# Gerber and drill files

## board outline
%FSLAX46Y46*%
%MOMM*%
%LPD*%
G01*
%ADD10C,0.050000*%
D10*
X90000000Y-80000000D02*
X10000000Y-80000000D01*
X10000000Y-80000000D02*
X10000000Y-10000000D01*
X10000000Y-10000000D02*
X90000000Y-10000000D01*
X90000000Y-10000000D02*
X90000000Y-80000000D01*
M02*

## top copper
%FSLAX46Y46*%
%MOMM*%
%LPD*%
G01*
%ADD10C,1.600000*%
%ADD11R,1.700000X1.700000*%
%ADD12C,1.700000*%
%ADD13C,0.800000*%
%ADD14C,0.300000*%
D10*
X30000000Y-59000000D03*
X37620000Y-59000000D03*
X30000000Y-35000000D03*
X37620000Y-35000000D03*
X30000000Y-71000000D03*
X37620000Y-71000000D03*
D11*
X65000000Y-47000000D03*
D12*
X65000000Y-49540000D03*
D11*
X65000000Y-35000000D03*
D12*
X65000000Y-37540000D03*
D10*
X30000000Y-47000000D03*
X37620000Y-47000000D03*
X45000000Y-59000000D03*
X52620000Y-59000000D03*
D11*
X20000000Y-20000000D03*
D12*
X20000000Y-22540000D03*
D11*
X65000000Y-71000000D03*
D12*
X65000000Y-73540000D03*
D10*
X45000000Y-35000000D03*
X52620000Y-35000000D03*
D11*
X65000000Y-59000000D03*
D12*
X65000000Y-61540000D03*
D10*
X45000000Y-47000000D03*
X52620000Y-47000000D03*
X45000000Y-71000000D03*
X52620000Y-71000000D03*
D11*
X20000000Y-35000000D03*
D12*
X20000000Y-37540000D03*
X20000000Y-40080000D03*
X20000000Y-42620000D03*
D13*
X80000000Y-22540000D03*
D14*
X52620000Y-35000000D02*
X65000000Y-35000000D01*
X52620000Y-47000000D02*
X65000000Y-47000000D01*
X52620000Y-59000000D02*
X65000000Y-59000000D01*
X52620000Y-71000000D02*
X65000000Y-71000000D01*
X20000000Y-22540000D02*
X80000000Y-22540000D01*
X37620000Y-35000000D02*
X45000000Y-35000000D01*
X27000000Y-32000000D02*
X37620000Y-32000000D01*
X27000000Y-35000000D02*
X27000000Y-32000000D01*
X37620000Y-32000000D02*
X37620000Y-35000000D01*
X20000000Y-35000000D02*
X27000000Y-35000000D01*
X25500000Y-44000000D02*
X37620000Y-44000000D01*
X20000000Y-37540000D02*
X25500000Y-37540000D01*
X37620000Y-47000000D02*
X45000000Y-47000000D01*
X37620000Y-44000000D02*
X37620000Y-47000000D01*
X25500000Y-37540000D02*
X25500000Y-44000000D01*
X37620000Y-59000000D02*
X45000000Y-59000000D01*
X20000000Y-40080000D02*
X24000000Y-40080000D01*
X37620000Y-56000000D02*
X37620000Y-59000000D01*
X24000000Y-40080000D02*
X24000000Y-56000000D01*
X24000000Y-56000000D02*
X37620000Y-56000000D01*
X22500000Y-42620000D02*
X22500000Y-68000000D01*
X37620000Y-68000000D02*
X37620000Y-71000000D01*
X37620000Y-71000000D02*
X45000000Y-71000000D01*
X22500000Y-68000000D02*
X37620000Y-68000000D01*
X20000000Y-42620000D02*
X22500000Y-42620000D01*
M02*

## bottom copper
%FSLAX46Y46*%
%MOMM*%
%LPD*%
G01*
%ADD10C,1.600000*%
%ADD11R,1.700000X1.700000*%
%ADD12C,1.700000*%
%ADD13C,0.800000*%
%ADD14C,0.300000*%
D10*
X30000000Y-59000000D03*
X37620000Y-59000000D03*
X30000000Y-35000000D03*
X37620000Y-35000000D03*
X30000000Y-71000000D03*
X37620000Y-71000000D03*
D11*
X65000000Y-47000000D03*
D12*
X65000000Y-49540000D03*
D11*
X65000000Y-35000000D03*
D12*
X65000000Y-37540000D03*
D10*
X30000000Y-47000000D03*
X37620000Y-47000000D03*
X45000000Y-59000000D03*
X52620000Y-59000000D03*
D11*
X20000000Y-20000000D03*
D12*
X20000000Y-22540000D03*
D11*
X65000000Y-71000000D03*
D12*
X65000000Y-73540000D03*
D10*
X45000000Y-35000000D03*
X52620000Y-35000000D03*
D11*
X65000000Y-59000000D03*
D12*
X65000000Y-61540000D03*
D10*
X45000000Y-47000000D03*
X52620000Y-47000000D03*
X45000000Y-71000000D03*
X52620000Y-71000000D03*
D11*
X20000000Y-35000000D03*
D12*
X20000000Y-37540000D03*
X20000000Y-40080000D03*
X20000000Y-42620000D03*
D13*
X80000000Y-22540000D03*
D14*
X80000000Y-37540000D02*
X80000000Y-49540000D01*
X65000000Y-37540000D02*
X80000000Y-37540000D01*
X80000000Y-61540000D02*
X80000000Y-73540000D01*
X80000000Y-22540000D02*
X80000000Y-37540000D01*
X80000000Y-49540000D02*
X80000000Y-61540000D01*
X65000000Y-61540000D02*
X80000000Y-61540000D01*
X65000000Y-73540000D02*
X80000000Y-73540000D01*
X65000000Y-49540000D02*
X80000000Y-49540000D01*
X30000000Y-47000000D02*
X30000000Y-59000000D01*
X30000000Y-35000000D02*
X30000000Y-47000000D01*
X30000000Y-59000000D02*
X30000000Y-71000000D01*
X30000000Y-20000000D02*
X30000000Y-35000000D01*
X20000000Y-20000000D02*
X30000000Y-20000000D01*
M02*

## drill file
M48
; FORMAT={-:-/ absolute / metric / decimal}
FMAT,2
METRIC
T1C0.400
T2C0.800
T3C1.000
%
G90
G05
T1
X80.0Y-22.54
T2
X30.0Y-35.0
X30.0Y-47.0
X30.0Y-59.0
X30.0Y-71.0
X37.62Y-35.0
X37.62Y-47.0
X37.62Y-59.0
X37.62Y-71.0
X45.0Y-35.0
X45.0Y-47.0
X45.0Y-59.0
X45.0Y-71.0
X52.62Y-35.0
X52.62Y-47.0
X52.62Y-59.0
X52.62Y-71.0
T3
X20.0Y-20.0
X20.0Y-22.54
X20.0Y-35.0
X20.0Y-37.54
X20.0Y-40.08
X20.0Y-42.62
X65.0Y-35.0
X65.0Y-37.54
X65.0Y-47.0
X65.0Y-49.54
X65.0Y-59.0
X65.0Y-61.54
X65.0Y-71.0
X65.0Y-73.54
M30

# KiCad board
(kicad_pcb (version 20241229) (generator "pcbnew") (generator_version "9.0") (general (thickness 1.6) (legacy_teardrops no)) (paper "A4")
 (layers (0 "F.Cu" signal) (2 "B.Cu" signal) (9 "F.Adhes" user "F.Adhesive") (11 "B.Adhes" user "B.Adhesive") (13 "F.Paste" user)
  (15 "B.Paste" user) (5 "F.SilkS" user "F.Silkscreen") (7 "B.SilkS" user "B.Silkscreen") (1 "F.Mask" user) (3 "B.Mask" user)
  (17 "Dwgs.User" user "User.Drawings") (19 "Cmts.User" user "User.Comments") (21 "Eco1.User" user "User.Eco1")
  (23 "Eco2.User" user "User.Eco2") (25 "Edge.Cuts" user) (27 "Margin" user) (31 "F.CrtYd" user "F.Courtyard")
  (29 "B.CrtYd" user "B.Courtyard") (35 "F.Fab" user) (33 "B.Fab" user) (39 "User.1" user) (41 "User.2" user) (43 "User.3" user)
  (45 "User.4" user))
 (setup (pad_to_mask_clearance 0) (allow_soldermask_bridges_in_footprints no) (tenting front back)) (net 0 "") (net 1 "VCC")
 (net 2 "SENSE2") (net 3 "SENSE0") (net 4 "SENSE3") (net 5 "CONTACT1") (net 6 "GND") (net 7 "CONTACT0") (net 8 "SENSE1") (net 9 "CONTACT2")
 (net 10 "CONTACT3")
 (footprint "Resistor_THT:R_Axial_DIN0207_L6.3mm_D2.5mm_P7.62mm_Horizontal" (layer "F.Cu") (at 30 59)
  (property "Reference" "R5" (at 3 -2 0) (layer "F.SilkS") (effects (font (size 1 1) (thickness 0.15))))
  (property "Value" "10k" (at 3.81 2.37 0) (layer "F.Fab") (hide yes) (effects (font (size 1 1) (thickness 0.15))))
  (pad "1" thru_hole circle (at 0 0) (size 1.6 1.6) (drill 0.8) (layers "*.Cu" "*.Mask") (remove_unused_layers no) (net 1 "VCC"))
  (pad "2" thru_hole circle (at 7.62 0) (size 1.6 1.6) (drill 0.8) (layers "*.Cu" "*.Mask") (remove_unused_layers no) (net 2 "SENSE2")))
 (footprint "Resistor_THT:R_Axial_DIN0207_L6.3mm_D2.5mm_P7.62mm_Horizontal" (layer "F.Cu") (at 30 35)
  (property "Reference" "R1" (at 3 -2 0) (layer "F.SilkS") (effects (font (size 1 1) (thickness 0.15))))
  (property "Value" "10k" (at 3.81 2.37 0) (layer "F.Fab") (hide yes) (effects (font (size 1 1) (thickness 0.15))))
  (pad "1" thru_hole circle (at 0 0) (size 1.6 1.6) (drill 0.8) (layers "*.Cu" "*.Mask") (remove_unused_layers no) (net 1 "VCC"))
  (pad "2" thru_hole circle (at 7.62 0) (size 1.6 1.6) (drill 0.8) (layers "*.Cu" "*.Mask") (remove_unused_layers no) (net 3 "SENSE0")))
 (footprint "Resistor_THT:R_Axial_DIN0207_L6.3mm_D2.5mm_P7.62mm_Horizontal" (layer "F.Cu") (at 30 71)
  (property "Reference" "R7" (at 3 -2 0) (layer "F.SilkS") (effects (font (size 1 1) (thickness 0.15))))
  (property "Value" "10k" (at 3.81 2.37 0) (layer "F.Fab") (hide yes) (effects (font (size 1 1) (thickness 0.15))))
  (pad "1" thru_hole circle (at 0 0) (size 1.6 1.6) (drill 0.8) (layers "*.Cu" "*.Mask") (remove_unused_layers no) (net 1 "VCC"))
  (pad "2" thru_hole circle (at 7.62 0) (size 1.6 1.6) (drill 0.8) (layers "*.Cu" "*.Mask") (remove_unused_layers no) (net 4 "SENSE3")))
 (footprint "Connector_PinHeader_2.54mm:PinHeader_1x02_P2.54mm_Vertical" (layer "F.Cu") (at 65 47)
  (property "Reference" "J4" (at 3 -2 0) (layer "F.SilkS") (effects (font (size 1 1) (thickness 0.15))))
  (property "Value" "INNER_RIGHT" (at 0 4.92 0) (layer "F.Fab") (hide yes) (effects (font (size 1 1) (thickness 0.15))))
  (pad "1" thru_hole rect (at 0 0) (size 1.7 1.7) (drill 1) (layers "*.Cu" "*.Mask") (remove_unused_layers no) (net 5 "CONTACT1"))
  (pad "2" thru_hole circle (at 0 2.54) (size 1.7 1.7) (drill 1) (layers "*.Cu" "*.Mask") (remove_unused_layers no) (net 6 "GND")))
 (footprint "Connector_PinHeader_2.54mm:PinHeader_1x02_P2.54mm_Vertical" (layer "F.Cu") (at 65 35)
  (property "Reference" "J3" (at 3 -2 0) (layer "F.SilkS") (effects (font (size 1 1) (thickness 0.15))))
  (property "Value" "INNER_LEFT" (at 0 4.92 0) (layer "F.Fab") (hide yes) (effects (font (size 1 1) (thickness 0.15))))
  (pad "1" thru_hole rect (at 0 0) (size 1.7 1.7) (drill 1) (layers "*.Cu" "*.Mask") (remove_unused_layers no) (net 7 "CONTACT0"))
  (pad "2" thru_hole circle (at 0 2.54) (size 1.7 1.7) (drill 1) (layers "*.Cu" "*.Mask") (remove_unused_layers no) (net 6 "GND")))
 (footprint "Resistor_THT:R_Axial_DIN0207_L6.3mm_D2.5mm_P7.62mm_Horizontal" (layer "F.Cu") (at 30 47)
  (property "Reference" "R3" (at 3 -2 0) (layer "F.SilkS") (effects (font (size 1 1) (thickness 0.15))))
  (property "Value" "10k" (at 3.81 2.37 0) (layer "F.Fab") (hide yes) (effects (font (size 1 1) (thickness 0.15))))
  (pad "1" thru_hole circle (at 0 0) (size 1.6 1.6) (drill 0.8) (layers "*.Cu" "*.Mask") (remove_unused_layers no) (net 1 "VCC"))
  (pad "2" thru_hole circle (at 7.62 0) (size 1.6 1.6) (drill 0.8) (layers "*.Cu" "*.Mask") (remove_unused_layers no) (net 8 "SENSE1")))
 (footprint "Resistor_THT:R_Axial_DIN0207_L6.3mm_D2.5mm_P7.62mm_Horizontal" (layer "F.Cu") (at 45 59)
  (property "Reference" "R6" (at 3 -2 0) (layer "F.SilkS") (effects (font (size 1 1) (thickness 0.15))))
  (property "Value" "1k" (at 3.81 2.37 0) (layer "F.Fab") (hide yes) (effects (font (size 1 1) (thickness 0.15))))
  (pad "1" thru_hole circle (at 0 0) (size 1.6 1.6) (drill 0.8) (layers "*.Cu" "*.Mask") (remove_unused_layers no) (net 2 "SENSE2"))
  (pad "2" thru_hole circle (at 7.62 0) (size 1.6 1.6) (drill 0.8) (layers "*.Cu" "*.Mask") (remove_unused_layers no) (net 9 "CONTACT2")))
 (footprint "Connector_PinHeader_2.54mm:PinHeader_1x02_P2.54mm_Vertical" (layer "F.Cu") (at 20 20)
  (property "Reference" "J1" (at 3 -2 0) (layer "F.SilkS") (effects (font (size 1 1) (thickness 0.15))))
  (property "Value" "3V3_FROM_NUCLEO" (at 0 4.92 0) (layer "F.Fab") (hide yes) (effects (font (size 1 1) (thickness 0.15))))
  (pad "1" thru_hole rect (at 0 0) (size 1.7 1.7) (drill 1) (layers "*.Cu" "*.Mask") (remove_unused_layers no) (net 1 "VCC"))
  (pad "2" thru_hole circle (at 0 2.54) (size 1.7 1.7) (drill 1) (layers "*.Cu" "*.Mask") (remove_unused_layers no) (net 6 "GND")))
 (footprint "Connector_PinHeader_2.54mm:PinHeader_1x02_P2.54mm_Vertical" (layer "F.Cu") (at 65 71)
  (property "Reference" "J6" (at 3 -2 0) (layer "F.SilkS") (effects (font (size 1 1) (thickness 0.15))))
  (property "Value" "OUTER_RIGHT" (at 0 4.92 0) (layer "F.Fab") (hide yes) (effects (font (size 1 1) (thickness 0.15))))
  (pad "1" thru_hole rect (at 0 0) (size 1.7 1.7) (drill 1) (layers "*.Cu" "*.Mask") (remove_unused_layers no) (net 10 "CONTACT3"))
  (pad "2" thru_hole circle (at 0 2.54) (size 1.7 1.7) (drill 1) (layers "*.Cu" "*.Mask") (remove_unused_layers no) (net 6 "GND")))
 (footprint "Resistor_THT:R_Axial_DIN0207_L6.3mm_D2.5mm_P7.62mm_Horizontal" (layer "F.Cu") (at 45 35)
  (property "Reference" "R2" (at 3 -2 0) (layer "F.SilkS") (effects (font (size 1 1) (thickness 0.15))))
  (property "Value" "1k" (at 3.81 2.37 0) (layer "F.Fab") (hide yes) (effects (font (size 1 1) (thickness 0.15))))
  (pad "1" thru_hole circle (at 0 0) (size 1.6 1.6) (drill 0.8) (layers "*.Cu" "*.Mask") (remove_unused_layers no) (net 3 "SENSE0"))
  (pad "2" thru_hole circle (at 7.62 0) (size 1.6 1.6) (drill 0.8) (layers "*.Cu" "*.Mask") (remove_unused_layers no) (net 7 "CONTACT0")))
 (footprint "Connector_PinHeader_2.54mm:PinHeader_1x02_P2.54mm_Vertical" (layer "F.Cu") (at 65 59)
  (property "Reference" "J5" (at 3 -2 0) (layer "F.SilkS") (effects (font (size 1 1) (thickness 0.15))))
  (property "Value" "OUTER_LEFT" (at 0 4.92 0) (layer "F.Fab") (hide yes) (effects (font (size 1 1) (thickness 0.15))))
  (pad "1" thru_hole rect (at 0 0) (size 1.7 1.7) (drill 1) (layers "*.Cu" "*.Mask") (remove_unused_layers no) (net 9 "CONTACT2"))
  (pad "2" thru_hole circle (at 0 2.54) (size 1.7 1.7) (drill 1) (layers "*.Cu" "*.Mask") (remove_unused_layers no) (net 6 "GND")))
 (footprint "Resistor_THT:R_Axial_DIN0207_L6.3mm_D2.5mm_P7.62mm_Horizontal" (layer "F.Cu") (at 45 47)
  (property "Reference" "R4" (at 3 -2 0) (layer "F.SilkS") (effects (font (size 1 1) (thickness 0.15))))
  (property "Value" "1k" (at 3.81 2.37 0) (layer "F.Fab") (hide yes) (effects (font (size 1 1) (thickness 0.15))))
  (pad "1" thru_hole circle (at 0 0) (size 1.6 1.6) (drill 0.8) (layers "*.Cu" "*.Mask") (remove_unused_layers no) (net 8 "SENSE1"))
  (pad "2" thru_hole circle (at 7.62 0) (size 1.6 1.6) (drill 0.8) (layers "*.Cu" "*.Mask") (remove_unused_layers no) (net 5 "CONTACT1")))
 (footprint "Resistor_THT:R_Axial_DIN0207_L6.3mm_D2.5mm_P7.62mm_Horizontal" (layer "F.Cu") (at 45 71)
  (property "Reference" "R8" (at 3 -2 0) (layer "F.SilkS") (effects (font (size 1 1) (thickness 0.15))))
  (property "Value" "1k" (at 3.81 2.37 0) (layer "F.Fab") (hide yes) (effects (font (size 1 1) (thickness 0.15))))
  (pad "1" thru_hole circle (at 0 0) (size 1.6 1.6) (drill 0.8) (layers "*.Cu" "*.Mask") (remove_unused_layers no) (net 4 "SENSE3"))
  (pad "2" thru_hole circle (at 7.62 0) (size 1.6 1.6) (drill 0.8) (layers "*.Cu" "*.Mask") (remove_unused_layers no) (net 10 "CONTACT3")))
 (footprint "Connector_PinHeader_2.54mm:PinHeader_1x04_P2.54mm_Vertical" (layer "F.Cu") (at 20 35)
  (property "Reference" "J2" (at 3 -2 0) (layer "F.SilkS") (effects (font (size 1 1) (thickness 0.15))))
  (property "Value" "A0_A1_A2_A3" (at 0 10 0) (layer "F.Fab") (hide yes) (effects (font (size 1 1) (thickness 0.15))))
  (pad "1" thru_hole rect (at 0 0) (size 1.7 1.7) (drill 1) (layers "*.Cu" "*.Mask") (remove_unused_layers no) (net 3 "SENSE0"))
  (pad "2" thru_hole circle (at 0 2.54) (size 1.7 1.7) (drill 1) (layers "*.Cu" "*.Mask") (remove_unused_layers no) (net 8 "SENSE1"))
  (pad "3" thru_hole circle (at 0 5.08) (size 1.7 1.7) (drill 1) (layers "*.Cu" "*.Mask") (remove_unused_layers no) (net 2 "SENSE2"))
  (pad "4" thru_hole circle (at 0 7.62) (size 1.7 1.7) (drill 1) (layers "*.Cu" "*.Mask") (remove_unused_layers no) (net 4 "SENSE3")))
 (gr_line (start 90 80) (end 10 80) (stroke (width 0.05) (type default)) (layer "Edge.Cuts"))
 (gr_line (start 10 80) (end 10 10) (stroke (width 0.05) (type default)) (layer "Edge.Cuts"))
 (gr_line (start 10 10) (end 90 10) (stroke (width 0.05) (type default)) (layer "Edge.Cuts"))
 (gr_line (start 90 10) (end 90 80) (stroke (width 0.05) (type default)) (layer "Edge.Cuts"))
 (segment (start 52.62 35) (end 65 35) (width 0.3) (layer "F.Cu") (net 7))
 (segment (start 52.62 47) (end 65 47) (width 0.3) (layer "F.Cu") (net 5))
 (segment (start 52.62 59) (end 65 59) (width 0.3) (layer "F.Cu") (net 9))
 (segment (start 52.62 71) (end 65 71) (width 0.3) (layer "F.Cu") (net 10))
 (segment (start 20 22.54) (end 80 22.54) (width 0.3) (layer "F.Cu") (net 6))
 (via (at 80 22.54) (size 0.8) (drill 0.4) (layers "F.Cu" "B.Cu") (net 6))
 (segment (start 80 37.54) (end 80 49.54) (width 0.3) (layer "B.Cu") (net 6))
 (segment (start 65 37.54) (end 80 37.54) (width 0.3) (layer "B.Cu") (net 6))
 (segment (start 80 61.54) (end 80 73.54) (width 0.3) (layer "B.Cu") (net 6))
 (segment (start 80 22.54) (end 80 37.54) (width 0.3) (layer "B.Cu") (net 6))
 (segment (start 80 49.54) (end 80 61.54) (width 0.3) (layer "B.Cu") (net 6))
 (segment (start 65 61.54) (end 80 61.54) (width 0.3) (layer "B.Cu") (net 6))
 (segment (start 65 73.54) (end 80 73.54) (width 0.3) (layer "B.Cu") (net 6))
 (segment (start 65 49.54) (end 80 49.54) (width 0.3) (layer "B.Cu") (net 6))
 (segment (start 37.62 35) (end 45 35) (width 0.3) (layer "F.Cu") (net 3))
 (segment (start 27 32) (end 37.62 32) (width 0.3) (layer "F.Cu") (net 3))
 (segment (start 27 35) (end 27 32) (width 0.3) (layer "F.Cu") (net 3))
 (segment (start 37.62 32) (end 37.62 35) (width 0.3) (layer "F.Cu") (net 3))
 (segment (start 20 35) (end 27 35) (width 0.3) (layer "F.Cu") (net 3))
 (segment (start 25.5 44) (end 37.62 44) (width 0.3) (layer "F.Cu") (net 8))
 (segment (start 20 37.54) (end 25.5 37.54) (width 0.3) (layer "F.Cu") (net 8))
 (segment (start 37.62 47) (end 45 47) (width 0.3) (layer "F.Cu") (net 8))
 (segment (start 37.62 44) (end 37.62 47) (width 0.3) (layer "F.Cu") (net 8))
 (segment (start 25.5 37.54) (end 25.5 44) (width 0.3) (layer "F.Cu") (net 8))
 (segment (start 37.62 59) (end 45 59) (width 0.3) (layer "F.Cu") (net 2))
 (segment (start 20 40.08) (end 24 40.08) (width 0.3) (layer "F.Cu") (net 2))
 (segment (start 37.62 56) (end 37.62 59) (width 0.3) (layer "F.Cu") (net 2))
 (segment (start 24 40.08) (end 24 56) (width 0.3) (layer "F.Cu") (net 2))
 (segment (start 24 56) (end 37.62 56) (width 0.3) (layer "F.Cu") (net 2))
 (segment (start 22.5 42.62) (end 22.5 68) (width 0.3) (layer "F.Cu") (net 4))
 (segment (start 37.62 68) (end 37.62 71) (width 0.3) (layer "F.Cu") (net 4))
 (segment (start 37.62 71) (end 45 71) (width 0.3) (layer "F.Cu") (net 4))
 (segment (start 22.5 68) (end 37.62 68) (width 0.3) (layer "F.Cu") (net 4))
 (segment (start 20 42.62) (end 22.5 42.62) (width 0.3) (layer "F.Cu") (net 4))
 (segment (start 30 47) (end 30 59) (width 0.3) (layer "B.Cu") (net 1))
 (segment (start 30 35) (end 30 47) (width 0.3) (layer "B.Cu") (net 1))
 (segment (start 30 59) (end 30 71) (width 0.3) (layer "B.Cu") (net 1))
 (segment (start 30 20) (end 30 35) (width 0.3) (layer "B.Cu") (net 1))
 (segment (start 20 20) (end 30 20) (width 0.3) (layer "B.Cu") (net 1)))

